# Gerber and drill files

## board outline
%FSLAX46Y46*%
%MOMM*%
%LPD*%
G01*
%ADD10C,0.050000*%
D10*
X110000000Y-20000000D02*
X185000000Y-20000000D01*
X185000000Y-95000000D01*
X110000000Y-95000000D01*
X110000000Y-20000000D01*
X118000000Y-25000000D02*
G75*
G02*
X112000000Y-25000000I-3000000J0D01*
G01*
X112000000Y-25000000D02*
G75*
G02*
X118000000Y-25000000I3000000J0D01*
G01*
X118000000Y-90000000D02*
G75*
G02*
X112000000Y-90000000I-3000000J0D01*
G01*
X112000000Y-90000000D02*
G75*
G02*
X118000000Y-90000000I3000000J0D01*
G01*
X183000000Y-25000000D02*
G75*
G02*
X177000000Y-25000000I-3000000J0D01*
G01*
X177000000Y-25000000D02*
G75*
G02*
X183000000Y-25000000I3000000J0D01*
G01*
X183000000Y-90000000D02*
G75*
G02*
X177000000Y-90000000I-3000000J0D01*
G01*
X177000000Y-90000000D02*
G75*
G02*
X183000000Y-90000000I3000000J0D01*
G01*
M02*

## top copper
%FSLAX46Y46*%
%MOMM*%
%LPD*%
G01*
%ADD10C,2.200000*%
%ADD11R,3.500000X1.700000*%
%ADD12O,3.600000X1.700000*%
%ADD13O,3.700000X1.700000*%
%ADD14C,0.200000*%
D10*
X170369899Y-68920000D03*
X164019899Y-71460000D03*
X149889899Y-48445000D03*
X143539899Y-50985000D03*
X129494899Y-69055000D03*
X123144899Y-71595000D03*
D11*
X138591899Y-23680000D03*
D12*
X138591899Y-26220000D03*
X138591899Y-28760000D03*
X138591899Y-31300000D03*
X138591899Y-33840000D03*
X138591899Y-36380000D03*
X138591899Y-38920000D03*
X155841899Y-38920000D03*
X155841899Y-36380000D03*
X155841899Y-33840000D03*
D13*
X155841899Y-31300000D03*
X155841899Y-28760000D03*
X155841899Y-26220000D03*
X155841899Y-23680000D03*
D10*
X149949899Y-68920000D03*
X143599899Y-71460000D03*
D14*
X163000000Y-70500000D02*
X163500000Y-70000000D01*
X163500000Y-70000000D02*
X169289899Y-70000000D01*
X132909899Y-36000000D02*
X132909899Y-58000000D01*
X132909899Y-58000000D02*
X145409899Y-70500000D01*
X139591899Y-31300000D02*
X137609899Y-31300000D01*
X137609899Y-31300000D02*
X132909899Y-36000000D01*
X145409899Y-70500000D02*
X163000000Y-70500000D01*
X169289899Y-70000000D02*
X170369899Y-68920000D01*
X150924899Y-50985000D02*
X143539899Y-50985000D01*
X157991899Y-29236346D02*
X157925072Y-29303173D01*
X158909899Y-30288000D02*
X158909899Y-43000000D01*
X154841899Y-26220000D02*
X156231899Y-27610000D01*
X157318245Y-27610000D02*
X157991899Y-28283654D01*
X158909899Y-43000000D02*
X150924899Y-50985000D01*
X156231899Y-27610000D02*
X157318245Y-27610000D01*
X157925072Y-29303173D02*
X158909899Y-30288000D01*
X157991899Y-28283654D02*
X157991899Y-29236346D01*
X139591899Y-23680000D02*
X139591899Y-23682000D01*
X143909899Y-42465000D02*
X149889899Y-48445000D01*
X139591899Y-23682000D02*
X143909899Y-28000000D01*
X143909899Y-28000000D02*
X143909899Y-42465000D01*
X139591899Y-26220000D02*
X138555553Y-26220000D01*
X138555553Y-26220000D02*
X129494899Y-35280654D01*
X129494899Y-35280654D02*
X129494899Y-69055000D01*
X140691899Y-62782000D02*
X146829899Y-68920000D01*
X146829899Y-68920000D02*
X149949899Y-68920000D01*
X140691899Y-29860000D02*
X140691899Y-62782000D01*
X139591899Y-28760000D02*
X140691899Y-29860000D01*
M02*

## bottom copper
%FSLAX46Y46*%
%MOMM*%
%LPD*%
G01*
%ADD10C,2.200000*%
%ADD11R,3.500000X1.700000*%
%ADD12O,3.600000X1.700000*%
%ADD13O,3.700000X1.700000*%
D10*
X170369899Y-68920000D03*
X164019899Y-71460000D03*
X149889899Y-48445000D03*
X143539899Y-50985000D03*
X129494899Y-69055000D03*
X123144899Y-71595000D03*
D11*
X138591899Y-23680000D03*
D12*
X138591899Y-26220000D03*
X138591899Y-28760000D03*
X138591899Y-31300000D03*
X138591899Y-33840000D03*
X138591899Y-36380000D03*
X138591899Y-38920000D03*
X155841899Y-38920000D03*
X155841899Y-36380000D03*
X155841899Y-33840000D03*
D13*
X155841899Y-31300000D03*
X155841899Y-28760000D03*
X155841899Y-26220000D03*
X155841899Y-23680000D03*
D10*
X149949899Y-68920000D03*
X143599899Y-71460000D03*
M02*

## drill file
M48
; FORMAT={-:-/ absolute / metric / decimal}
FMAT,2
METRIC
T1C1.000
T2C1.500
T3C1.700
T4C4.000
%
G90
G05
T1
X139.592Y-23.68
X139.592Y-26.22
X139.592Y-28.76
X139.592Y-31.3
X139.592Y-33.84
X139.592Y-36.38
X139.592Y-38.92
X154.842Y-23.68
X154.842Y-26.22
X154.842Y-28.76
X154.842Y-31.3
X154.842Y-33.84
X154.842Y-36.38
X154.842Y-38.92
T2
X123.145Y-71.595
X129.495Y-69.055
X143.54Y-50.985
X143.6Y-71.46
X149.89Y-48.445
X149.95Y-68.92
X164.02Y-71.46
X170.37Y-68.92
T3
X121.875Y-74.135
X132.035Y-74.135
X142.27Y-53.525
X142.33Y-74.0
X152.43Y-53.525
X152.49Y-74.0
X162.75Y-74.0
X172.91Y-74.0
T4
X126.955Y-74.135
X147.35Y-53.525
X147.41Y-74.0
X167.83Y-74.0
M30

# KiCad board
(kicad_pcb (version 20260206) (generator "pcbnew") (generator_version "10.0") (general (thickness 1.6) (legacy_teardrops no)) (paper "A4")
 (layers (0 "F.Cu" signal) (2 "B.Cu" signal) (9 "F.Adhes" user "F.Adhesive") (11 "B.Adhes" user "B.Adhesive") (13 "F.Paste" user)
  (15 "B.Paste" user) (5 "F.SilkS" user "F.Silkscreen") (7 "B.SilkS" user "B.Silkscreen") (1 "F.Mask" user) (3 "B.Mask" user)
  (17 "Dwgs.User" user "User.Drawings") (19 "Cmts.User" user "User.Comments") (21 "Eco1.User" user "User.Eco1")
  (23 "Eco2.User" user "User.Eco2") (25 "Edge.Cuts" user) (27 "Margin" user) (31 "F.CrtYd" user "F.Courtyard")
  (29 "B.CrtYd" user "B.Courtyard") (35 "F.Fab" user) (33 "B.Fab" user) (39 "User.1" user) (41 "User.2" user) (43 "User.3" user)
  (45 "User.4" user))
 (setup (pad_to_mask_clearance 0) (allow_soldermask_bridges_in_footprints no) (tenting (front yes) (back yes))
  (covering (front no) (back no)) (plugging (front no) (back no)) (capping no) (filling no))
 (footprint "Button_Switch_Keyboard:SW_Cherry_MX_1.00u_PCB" (layer "F.Cu") (at 170.369899 68.92)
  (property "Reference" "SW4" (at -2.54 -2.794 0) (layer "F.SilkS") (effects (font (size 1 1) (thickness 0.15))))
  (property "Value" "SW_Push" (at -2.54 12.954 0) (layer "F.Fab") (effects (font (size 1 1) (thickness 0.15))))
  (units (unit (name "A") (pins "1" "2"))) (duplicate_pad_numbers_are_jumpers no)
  (pad "" np_thru_hole circle (at -7.62 5.08) (size 1.7 1.7) (drill 1.7) (layers "*.Cu" "*.Mask"))
  (pad "" np_thru_hole circle (at -2.54 5.08) (size 4 4) (drill 4) (layers "*.Cu" "*.Mask"))
  (pad "" np_thru_hole circle (at 2.54 5.08) (size 1.7 1.7) (drill 1.7) (layers "*.Cu" "*.Mask"))
  (pad "1" thru_hole circle (at 0 0) (size 2.2 2.2) (drill 1.5) (layers "*.Cu" "*.Mask") (remove_unused_layers no)
   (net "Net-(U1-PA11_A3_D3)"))
  (pad "2" thru_hole circle (at -6.35 2.54) (size 2.2 2.2) (drill 1.5) (layers "*.Cu" "*.Mask") (remove_unused_layers no) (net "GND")))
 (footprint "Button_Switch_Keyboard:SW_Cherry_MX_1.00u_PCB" (layer "F.Cu") (at 149.889899 48.445)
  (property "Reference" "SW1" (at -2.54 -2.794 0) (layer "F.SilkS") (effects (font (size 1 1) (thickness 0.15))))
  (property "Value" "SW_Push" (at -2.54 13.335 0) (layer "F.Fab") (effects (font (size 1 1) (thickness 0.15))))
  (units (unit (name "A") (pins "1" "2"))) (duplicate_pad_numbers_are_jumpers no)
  (pad "" np_thru_hole circle (at -7.62 5.08) (size 1.7 1.7) (drill 1.7) (layers "*.Cu" "*.Mask"))
  (pad "" np_thru_hole circle (at -2.54 5.08) (size 4 4) (drill 4) (layers "*.Cu" "*.Mask"))
  (pad "" np_thru_hole circle (at 2.54 5.08) (size 1.7 1.7) (drill 1.7) (layers "*.Cu" "*.Mask"))
  (pad "1" thru_hole circle (at 0 0) (size 2.2 2.2) (drill 1.5) (layers "*.Cu" "*.Mask") (remove_unused_layers no)
   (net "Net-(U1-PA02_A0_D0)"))
  (pad "2" thru_hole circle (at -6.35 2.54) (size 2.2 2.2) (drill 1.5) (layers "*.Cu" "*.Mask") (remove_unused_layers no) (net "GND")))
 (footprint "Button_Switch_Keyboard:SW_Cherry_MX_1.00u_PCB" (layer "F.Cu") (at 129.494899 69.055)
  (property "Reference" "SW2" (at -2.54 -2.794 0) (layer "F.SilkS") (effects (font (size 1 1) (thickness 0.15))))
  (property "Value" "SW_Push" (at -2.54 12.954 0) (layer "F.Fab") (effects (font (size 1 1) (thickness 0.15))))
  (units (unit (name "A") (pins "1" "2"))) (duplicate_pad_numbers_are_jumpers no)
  (pad "" np_thru_hole circle (at -7.62 5.08) (size 1.7 1.7) (drill 1.7) (layers "*.Cu" "*.Mask"))
  (pad "" np_thru_hole circle (at -2.54 5.08) (size 4 4) (drill 4) (layers "*.Cu" "*.Mask"))
  (pad "" np_thru_hole circle (at 2.54 5.08) (size 1.7 1.7) (drill 1.7) (layers "*.Cu" "*.Mask"))
  (pad "1" thru_hole circle (at 0 0) (size 2.2 2.2) (drill 1.5) (layers "*.Cu" "*.Mask") (remove_unused_layers no)
   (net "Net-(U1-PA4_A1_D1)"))
  (pad "2" thru_hole circle (at -6.35 2.54) (size 2.2 2.2) (drill 1.5) (layers "*.Cu" "*.Mask") (remove_unused_layers no) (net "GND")))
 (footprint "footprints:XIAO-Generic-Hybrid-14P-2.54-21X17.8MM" (layer "F.Cu") (at 147.216899 31.3)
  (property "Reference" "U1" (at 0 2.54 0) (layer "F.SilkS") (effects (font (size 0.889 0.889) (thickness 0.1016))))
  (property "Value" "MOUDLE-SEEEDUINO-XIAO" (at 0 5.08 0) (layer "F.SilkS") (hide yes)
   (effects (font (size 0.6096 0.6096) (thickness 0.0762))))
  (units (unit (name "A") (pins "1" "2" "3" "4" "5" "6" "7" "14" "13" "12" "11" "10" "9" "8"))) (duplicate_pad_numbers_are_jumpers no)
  (pad "1" thru_hole rect (at -7.625 -7.62) (size 3.5 1.7) (drill 1 (offset -1 0)) (layers "*.Cu" "*.Mask") (remove_unused_layers no)
   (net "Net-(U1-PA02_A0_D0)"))
  (pad "2" thru_hole oval (at -7.625 -5.08) (size 3.6 1.7) (drill 1 (offset -1 0)) (layers "*.Cu" "*.Mask") (remove_unused_layers no)
   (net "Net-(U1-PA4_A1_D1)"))
  (pad "3" thru_hole oval (at -7.625 -2.54) (size 3.6 1.7) (drill 1 (offset -1 0)) (layers "*.Cu" "*.Mask") (remove_unused_layers no)
   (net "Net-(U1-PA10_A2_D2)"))
  (pad "4" thru_hole oval (at -7.625 0) (size 3.6 1.7) (drill 1 (offset -1 0)) (layers "*.Cu" "*.Mask") (remove_unused_layers no)
   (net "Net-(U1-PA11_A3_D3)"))
  (pad "5" thru_hole oval (at -7.625 2.54) (size 3.6 1.7) (drill 1 (offset -1 0)) (layers "*.Cu" "*.Mask") (remove_unused_layers no)
   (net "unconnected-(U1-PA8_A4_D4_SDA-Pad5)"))
  (pad "6" thru_hole oval (at -7.625 5.08 180) (size 3.6 1.7) (drill 1 (offset 1 0)) (layers "*.Cu" "*.Mask") (remove_unused_layers no)
   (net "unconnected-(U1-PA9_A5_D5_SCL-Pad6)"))
  (pad "7" thru_hole oval (at -7.625 7.62) (size 3.6 1.7) (drill 1 (offset -1 0)) (layers "*.Cu" "*.Mask") (remove_unused_layers no)
   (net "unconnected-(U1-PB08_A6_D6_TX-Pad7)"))
  (pad "8" thru_hole oval (at 7.625 7.62) (size 3.6 1.7) (drill 1 (offset 1 0)) (layers "*.Cu" "*.Mask") (remove_unused_layers no)
   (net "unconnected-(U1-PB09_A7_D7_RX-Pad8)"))
  (pad "9" thru_hole oval (at 7.625 5.08) (size 3.6 1.7) (drill 1 (offset 1 0)) (layers "*.Cu" "*.Mask") (remove_unused_layers no)
   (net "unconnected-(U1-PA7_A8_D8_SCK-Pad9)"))
  (pad "10" thru_hole oval (at 7.625 2.54) (size 3.6 1.7) (drill 1 (offset 1 0)) (layers "*.Cu" "*.Mask") (remove_unused_layers no)
   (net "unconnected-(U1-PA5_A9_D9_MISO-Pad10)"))
  (pad "11" thru_hole oval (at 7.625 0) (size 3.7 1.7) (drill 1 (offset 1 0)) (layers "*.Cu" "*.Mask") (remove_unused_layers no)
   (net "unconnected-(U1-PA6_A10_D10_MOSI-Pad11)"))
  (pad "12" thru_hole oval (at 7.625 -2.54) (size 3.7 1.7) (drill 1 (offset 1 0)) (layers "*.Cu" "*.Mask") (remove_unused_layers no)
   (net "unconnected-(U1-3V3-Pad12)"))
  (pad "13" thru_hole oval (at 7.625 -5.08) (size 3.7 1.7) (drill 1 (offset 1 0)) (layers "*.Cu" "*.Mask") (remove_unused_layers no)
   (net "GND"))
  (pad "14" thru_hole oval (at 7.625 -7.62) (size 3.7 1.7) (drill 1 (offset 1 0)) (layers "*.Cu" "*.Mask") (remove_unused_layers no)
   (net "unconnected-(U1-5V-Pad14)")))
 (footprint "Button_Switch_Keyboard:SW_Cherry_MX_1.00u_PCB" (layer "F.Cu") (at 149.949899 68.92)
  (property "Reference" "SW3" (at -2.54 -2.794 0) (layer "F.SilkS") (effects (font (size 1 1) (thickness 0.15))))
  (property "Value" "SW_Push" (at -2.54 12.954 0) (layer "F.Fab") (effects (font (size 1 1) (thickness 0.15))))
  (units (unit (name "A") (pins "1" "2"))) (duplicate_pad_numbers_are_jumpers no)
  (pad "" np_thru_hole circle (at -7.62 5.08) (size 1.7 1.7) (drill 1.7) (layers "*.Cu" "*.Mask"))
  (pad "" np_thru_hole circle (at -2.54 5.08) (size 4 4) (drill 4) (layers "*.Cu" "*.Mask"))
  (pad "" np_thru_hole circle (at 2.54 5.08) (size 1.7 1.7) (drill 1.7) (layers "*.Cu" "*.Mask"))
  (pad "1" thru_hole circle (at 0 0) (size 2.2 2.2) (drill 1.5) (layers "*.Cu" "*.Mask") (remove_unused_layers no)
   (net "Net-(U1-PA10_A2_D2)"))
  (pad "2" thru_hole circle (at -6.35 2.54) (size 2.2 2.2) (drill 1.5) (layers "*.Cu" "*.Mask") (remove_unused_layers no) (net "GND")))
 (gr_rect (start 110 20) (end 185 95) (stroke (width 0.05) (type default)) (fill no) (layer "Edge.Cuts"))
 (gr_circle (center 115 25) (end 118 25) (stroke (width 0.05) (type default)) (fill no) (layer "Edge.Cuts"))
 (gr_circle (center 115 90) (end 118 90) (stroke (width 0.05) (type default)) (fill no) (layer "Edge.Cuts"))
 (gr_circle (center 180 25) (end 177 25) (stroke (width 0.05) (type default)) (fill no) (layer "Edge.Cuts"))
 (gr_circle (center 180 90) (end 177 90) (stroke (width 0.05) (type default)) (fill no) (layer "Edge.Cuts"))
 (segment (start 163 70.5) (end 163.5 70) (width 0.2) (layer "F.Cu") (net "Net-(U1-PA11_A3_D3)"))
 (segment (start 163.5 70) (end 169.289899 70) (width 0.2) (layer "F.Cu") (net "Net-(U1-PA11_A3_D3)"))
 (segment (start 132.909899 36) (end 132.909899 58) (width 0.2) (layer "F.Cu") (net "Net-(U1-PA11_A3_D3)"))
 (segment (start 132.909899 58) (end 145.409899 70.5) (width 0.2) (layer "F.Cu") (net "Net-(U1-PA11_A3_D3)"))
 (segment (start 139.591899 31.3) (end 137.609899 31.3) (width 0.2) (layer "F.Cu") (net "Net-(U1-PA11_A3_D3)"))
 (segment (start 137.609899 31.3) (end 132.909899 36) (width 0.2) (layer "F.Cu") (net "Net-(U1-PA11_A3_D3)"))
 (segment (start 145.409899 70.5) (end 163 70.5) (width 0.2) (layer "F.Cu") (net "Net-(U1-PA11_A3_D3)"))
 (segment (start 169.289899 70) (end 170.369899 68.92) (width 0.2) (layer "F.Cu") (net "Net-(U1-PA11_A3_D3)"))
 (segment (start 150.924899 50.985) (end 143.539899 50.985) (width 0.2) (layer "F.Cu") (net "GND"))
 (segment (start 157.991899 29.236346) (end 157.925072 29.303173) (width 0.2) (layer "F.Cu") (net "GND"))
 (segment (start 158.909899 30.288) (end 158.909899 43) (width 0.2) (layer "F.Cu") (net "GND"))
 (segment (start 154.841899 26.22) (end 156.231899 27.61) (width 0.2) (layer "F.Cu") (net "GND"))
 (segment (start 157.318245 27.61) (end 157.991899 28.283654) (width 0.2) (layer "F.Cu") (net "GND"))
 (segment (start 158.909899 43) (end 150.924899 50.985) (width 0.2) (layer "F.Cu") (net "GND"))
 (segment (start 156.231899 27.61) (end 157.318245 27.61) (width 0.2) (layer "F.Cu") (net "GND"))
 (segment (start 157.925072 29.303173) (end 158.909899 30.288) (width 0.2) (layer "F.Cu") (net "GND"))
 (segment (start 157.991899 28.283654) (end 157.991899 29.236346) (width 0.2) (layer "F.Cu") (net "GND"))
 (segment (start 139.591899 23.68) (end 139.591899 23.682) (width 0.2) (layer "F.Cu") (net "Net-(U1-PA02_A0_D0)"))
 (segment (start 143.909899 42.465) (end 149.889899 48.445) (width 0.2) (layer "F.Cu") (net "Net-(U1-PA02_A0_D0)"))
 (segment (start 139.591899 23.682) (end 143.909899 28) (width 0.2) (layer "F.Cu") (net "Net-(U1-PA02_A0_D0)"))
 (segment (start 143.909899 28) (end 143.909899 42.465) (width 0.2) (layer "F.Cu") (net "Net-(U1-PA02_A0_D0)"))
 (segment (start 139.591899 26.22) (end 138.555553 26.22) (width 0.2) (layer "F.Cu") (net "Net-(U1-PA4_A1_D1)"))
 (segment (start 138.555553 26.22) (end 129.494899 35.280654) (width 0.2) (layer "F.Cu") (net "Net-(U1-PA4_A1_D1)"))
 (segment (start 129.494899 35.280654) (end 129.494899 69.055) (width 0.2) (layer "F.Cu") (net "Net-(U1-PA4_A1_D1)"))
 (segment (start 140.691899 62.782) (end 146.829899 68.92) (width 0.2) (layer "F.Cu") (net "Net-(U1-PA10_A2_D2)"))
 (segment (start 146.829899 68.92) (end 149.949899 68.92) (width 0.2) (layer "F.Cu") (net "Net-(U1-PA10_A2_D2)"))
 (segment (start 140.691899 29.86) (end 140.691899 62.782) (width 0.2) (layer "F.Cu") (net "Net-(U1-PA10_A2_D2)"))
 (segment (start 139.591899 28.76) (end 140.691899 29.86) (width 0.2) (layer "F.Cu") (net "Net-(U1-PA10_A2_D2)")))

